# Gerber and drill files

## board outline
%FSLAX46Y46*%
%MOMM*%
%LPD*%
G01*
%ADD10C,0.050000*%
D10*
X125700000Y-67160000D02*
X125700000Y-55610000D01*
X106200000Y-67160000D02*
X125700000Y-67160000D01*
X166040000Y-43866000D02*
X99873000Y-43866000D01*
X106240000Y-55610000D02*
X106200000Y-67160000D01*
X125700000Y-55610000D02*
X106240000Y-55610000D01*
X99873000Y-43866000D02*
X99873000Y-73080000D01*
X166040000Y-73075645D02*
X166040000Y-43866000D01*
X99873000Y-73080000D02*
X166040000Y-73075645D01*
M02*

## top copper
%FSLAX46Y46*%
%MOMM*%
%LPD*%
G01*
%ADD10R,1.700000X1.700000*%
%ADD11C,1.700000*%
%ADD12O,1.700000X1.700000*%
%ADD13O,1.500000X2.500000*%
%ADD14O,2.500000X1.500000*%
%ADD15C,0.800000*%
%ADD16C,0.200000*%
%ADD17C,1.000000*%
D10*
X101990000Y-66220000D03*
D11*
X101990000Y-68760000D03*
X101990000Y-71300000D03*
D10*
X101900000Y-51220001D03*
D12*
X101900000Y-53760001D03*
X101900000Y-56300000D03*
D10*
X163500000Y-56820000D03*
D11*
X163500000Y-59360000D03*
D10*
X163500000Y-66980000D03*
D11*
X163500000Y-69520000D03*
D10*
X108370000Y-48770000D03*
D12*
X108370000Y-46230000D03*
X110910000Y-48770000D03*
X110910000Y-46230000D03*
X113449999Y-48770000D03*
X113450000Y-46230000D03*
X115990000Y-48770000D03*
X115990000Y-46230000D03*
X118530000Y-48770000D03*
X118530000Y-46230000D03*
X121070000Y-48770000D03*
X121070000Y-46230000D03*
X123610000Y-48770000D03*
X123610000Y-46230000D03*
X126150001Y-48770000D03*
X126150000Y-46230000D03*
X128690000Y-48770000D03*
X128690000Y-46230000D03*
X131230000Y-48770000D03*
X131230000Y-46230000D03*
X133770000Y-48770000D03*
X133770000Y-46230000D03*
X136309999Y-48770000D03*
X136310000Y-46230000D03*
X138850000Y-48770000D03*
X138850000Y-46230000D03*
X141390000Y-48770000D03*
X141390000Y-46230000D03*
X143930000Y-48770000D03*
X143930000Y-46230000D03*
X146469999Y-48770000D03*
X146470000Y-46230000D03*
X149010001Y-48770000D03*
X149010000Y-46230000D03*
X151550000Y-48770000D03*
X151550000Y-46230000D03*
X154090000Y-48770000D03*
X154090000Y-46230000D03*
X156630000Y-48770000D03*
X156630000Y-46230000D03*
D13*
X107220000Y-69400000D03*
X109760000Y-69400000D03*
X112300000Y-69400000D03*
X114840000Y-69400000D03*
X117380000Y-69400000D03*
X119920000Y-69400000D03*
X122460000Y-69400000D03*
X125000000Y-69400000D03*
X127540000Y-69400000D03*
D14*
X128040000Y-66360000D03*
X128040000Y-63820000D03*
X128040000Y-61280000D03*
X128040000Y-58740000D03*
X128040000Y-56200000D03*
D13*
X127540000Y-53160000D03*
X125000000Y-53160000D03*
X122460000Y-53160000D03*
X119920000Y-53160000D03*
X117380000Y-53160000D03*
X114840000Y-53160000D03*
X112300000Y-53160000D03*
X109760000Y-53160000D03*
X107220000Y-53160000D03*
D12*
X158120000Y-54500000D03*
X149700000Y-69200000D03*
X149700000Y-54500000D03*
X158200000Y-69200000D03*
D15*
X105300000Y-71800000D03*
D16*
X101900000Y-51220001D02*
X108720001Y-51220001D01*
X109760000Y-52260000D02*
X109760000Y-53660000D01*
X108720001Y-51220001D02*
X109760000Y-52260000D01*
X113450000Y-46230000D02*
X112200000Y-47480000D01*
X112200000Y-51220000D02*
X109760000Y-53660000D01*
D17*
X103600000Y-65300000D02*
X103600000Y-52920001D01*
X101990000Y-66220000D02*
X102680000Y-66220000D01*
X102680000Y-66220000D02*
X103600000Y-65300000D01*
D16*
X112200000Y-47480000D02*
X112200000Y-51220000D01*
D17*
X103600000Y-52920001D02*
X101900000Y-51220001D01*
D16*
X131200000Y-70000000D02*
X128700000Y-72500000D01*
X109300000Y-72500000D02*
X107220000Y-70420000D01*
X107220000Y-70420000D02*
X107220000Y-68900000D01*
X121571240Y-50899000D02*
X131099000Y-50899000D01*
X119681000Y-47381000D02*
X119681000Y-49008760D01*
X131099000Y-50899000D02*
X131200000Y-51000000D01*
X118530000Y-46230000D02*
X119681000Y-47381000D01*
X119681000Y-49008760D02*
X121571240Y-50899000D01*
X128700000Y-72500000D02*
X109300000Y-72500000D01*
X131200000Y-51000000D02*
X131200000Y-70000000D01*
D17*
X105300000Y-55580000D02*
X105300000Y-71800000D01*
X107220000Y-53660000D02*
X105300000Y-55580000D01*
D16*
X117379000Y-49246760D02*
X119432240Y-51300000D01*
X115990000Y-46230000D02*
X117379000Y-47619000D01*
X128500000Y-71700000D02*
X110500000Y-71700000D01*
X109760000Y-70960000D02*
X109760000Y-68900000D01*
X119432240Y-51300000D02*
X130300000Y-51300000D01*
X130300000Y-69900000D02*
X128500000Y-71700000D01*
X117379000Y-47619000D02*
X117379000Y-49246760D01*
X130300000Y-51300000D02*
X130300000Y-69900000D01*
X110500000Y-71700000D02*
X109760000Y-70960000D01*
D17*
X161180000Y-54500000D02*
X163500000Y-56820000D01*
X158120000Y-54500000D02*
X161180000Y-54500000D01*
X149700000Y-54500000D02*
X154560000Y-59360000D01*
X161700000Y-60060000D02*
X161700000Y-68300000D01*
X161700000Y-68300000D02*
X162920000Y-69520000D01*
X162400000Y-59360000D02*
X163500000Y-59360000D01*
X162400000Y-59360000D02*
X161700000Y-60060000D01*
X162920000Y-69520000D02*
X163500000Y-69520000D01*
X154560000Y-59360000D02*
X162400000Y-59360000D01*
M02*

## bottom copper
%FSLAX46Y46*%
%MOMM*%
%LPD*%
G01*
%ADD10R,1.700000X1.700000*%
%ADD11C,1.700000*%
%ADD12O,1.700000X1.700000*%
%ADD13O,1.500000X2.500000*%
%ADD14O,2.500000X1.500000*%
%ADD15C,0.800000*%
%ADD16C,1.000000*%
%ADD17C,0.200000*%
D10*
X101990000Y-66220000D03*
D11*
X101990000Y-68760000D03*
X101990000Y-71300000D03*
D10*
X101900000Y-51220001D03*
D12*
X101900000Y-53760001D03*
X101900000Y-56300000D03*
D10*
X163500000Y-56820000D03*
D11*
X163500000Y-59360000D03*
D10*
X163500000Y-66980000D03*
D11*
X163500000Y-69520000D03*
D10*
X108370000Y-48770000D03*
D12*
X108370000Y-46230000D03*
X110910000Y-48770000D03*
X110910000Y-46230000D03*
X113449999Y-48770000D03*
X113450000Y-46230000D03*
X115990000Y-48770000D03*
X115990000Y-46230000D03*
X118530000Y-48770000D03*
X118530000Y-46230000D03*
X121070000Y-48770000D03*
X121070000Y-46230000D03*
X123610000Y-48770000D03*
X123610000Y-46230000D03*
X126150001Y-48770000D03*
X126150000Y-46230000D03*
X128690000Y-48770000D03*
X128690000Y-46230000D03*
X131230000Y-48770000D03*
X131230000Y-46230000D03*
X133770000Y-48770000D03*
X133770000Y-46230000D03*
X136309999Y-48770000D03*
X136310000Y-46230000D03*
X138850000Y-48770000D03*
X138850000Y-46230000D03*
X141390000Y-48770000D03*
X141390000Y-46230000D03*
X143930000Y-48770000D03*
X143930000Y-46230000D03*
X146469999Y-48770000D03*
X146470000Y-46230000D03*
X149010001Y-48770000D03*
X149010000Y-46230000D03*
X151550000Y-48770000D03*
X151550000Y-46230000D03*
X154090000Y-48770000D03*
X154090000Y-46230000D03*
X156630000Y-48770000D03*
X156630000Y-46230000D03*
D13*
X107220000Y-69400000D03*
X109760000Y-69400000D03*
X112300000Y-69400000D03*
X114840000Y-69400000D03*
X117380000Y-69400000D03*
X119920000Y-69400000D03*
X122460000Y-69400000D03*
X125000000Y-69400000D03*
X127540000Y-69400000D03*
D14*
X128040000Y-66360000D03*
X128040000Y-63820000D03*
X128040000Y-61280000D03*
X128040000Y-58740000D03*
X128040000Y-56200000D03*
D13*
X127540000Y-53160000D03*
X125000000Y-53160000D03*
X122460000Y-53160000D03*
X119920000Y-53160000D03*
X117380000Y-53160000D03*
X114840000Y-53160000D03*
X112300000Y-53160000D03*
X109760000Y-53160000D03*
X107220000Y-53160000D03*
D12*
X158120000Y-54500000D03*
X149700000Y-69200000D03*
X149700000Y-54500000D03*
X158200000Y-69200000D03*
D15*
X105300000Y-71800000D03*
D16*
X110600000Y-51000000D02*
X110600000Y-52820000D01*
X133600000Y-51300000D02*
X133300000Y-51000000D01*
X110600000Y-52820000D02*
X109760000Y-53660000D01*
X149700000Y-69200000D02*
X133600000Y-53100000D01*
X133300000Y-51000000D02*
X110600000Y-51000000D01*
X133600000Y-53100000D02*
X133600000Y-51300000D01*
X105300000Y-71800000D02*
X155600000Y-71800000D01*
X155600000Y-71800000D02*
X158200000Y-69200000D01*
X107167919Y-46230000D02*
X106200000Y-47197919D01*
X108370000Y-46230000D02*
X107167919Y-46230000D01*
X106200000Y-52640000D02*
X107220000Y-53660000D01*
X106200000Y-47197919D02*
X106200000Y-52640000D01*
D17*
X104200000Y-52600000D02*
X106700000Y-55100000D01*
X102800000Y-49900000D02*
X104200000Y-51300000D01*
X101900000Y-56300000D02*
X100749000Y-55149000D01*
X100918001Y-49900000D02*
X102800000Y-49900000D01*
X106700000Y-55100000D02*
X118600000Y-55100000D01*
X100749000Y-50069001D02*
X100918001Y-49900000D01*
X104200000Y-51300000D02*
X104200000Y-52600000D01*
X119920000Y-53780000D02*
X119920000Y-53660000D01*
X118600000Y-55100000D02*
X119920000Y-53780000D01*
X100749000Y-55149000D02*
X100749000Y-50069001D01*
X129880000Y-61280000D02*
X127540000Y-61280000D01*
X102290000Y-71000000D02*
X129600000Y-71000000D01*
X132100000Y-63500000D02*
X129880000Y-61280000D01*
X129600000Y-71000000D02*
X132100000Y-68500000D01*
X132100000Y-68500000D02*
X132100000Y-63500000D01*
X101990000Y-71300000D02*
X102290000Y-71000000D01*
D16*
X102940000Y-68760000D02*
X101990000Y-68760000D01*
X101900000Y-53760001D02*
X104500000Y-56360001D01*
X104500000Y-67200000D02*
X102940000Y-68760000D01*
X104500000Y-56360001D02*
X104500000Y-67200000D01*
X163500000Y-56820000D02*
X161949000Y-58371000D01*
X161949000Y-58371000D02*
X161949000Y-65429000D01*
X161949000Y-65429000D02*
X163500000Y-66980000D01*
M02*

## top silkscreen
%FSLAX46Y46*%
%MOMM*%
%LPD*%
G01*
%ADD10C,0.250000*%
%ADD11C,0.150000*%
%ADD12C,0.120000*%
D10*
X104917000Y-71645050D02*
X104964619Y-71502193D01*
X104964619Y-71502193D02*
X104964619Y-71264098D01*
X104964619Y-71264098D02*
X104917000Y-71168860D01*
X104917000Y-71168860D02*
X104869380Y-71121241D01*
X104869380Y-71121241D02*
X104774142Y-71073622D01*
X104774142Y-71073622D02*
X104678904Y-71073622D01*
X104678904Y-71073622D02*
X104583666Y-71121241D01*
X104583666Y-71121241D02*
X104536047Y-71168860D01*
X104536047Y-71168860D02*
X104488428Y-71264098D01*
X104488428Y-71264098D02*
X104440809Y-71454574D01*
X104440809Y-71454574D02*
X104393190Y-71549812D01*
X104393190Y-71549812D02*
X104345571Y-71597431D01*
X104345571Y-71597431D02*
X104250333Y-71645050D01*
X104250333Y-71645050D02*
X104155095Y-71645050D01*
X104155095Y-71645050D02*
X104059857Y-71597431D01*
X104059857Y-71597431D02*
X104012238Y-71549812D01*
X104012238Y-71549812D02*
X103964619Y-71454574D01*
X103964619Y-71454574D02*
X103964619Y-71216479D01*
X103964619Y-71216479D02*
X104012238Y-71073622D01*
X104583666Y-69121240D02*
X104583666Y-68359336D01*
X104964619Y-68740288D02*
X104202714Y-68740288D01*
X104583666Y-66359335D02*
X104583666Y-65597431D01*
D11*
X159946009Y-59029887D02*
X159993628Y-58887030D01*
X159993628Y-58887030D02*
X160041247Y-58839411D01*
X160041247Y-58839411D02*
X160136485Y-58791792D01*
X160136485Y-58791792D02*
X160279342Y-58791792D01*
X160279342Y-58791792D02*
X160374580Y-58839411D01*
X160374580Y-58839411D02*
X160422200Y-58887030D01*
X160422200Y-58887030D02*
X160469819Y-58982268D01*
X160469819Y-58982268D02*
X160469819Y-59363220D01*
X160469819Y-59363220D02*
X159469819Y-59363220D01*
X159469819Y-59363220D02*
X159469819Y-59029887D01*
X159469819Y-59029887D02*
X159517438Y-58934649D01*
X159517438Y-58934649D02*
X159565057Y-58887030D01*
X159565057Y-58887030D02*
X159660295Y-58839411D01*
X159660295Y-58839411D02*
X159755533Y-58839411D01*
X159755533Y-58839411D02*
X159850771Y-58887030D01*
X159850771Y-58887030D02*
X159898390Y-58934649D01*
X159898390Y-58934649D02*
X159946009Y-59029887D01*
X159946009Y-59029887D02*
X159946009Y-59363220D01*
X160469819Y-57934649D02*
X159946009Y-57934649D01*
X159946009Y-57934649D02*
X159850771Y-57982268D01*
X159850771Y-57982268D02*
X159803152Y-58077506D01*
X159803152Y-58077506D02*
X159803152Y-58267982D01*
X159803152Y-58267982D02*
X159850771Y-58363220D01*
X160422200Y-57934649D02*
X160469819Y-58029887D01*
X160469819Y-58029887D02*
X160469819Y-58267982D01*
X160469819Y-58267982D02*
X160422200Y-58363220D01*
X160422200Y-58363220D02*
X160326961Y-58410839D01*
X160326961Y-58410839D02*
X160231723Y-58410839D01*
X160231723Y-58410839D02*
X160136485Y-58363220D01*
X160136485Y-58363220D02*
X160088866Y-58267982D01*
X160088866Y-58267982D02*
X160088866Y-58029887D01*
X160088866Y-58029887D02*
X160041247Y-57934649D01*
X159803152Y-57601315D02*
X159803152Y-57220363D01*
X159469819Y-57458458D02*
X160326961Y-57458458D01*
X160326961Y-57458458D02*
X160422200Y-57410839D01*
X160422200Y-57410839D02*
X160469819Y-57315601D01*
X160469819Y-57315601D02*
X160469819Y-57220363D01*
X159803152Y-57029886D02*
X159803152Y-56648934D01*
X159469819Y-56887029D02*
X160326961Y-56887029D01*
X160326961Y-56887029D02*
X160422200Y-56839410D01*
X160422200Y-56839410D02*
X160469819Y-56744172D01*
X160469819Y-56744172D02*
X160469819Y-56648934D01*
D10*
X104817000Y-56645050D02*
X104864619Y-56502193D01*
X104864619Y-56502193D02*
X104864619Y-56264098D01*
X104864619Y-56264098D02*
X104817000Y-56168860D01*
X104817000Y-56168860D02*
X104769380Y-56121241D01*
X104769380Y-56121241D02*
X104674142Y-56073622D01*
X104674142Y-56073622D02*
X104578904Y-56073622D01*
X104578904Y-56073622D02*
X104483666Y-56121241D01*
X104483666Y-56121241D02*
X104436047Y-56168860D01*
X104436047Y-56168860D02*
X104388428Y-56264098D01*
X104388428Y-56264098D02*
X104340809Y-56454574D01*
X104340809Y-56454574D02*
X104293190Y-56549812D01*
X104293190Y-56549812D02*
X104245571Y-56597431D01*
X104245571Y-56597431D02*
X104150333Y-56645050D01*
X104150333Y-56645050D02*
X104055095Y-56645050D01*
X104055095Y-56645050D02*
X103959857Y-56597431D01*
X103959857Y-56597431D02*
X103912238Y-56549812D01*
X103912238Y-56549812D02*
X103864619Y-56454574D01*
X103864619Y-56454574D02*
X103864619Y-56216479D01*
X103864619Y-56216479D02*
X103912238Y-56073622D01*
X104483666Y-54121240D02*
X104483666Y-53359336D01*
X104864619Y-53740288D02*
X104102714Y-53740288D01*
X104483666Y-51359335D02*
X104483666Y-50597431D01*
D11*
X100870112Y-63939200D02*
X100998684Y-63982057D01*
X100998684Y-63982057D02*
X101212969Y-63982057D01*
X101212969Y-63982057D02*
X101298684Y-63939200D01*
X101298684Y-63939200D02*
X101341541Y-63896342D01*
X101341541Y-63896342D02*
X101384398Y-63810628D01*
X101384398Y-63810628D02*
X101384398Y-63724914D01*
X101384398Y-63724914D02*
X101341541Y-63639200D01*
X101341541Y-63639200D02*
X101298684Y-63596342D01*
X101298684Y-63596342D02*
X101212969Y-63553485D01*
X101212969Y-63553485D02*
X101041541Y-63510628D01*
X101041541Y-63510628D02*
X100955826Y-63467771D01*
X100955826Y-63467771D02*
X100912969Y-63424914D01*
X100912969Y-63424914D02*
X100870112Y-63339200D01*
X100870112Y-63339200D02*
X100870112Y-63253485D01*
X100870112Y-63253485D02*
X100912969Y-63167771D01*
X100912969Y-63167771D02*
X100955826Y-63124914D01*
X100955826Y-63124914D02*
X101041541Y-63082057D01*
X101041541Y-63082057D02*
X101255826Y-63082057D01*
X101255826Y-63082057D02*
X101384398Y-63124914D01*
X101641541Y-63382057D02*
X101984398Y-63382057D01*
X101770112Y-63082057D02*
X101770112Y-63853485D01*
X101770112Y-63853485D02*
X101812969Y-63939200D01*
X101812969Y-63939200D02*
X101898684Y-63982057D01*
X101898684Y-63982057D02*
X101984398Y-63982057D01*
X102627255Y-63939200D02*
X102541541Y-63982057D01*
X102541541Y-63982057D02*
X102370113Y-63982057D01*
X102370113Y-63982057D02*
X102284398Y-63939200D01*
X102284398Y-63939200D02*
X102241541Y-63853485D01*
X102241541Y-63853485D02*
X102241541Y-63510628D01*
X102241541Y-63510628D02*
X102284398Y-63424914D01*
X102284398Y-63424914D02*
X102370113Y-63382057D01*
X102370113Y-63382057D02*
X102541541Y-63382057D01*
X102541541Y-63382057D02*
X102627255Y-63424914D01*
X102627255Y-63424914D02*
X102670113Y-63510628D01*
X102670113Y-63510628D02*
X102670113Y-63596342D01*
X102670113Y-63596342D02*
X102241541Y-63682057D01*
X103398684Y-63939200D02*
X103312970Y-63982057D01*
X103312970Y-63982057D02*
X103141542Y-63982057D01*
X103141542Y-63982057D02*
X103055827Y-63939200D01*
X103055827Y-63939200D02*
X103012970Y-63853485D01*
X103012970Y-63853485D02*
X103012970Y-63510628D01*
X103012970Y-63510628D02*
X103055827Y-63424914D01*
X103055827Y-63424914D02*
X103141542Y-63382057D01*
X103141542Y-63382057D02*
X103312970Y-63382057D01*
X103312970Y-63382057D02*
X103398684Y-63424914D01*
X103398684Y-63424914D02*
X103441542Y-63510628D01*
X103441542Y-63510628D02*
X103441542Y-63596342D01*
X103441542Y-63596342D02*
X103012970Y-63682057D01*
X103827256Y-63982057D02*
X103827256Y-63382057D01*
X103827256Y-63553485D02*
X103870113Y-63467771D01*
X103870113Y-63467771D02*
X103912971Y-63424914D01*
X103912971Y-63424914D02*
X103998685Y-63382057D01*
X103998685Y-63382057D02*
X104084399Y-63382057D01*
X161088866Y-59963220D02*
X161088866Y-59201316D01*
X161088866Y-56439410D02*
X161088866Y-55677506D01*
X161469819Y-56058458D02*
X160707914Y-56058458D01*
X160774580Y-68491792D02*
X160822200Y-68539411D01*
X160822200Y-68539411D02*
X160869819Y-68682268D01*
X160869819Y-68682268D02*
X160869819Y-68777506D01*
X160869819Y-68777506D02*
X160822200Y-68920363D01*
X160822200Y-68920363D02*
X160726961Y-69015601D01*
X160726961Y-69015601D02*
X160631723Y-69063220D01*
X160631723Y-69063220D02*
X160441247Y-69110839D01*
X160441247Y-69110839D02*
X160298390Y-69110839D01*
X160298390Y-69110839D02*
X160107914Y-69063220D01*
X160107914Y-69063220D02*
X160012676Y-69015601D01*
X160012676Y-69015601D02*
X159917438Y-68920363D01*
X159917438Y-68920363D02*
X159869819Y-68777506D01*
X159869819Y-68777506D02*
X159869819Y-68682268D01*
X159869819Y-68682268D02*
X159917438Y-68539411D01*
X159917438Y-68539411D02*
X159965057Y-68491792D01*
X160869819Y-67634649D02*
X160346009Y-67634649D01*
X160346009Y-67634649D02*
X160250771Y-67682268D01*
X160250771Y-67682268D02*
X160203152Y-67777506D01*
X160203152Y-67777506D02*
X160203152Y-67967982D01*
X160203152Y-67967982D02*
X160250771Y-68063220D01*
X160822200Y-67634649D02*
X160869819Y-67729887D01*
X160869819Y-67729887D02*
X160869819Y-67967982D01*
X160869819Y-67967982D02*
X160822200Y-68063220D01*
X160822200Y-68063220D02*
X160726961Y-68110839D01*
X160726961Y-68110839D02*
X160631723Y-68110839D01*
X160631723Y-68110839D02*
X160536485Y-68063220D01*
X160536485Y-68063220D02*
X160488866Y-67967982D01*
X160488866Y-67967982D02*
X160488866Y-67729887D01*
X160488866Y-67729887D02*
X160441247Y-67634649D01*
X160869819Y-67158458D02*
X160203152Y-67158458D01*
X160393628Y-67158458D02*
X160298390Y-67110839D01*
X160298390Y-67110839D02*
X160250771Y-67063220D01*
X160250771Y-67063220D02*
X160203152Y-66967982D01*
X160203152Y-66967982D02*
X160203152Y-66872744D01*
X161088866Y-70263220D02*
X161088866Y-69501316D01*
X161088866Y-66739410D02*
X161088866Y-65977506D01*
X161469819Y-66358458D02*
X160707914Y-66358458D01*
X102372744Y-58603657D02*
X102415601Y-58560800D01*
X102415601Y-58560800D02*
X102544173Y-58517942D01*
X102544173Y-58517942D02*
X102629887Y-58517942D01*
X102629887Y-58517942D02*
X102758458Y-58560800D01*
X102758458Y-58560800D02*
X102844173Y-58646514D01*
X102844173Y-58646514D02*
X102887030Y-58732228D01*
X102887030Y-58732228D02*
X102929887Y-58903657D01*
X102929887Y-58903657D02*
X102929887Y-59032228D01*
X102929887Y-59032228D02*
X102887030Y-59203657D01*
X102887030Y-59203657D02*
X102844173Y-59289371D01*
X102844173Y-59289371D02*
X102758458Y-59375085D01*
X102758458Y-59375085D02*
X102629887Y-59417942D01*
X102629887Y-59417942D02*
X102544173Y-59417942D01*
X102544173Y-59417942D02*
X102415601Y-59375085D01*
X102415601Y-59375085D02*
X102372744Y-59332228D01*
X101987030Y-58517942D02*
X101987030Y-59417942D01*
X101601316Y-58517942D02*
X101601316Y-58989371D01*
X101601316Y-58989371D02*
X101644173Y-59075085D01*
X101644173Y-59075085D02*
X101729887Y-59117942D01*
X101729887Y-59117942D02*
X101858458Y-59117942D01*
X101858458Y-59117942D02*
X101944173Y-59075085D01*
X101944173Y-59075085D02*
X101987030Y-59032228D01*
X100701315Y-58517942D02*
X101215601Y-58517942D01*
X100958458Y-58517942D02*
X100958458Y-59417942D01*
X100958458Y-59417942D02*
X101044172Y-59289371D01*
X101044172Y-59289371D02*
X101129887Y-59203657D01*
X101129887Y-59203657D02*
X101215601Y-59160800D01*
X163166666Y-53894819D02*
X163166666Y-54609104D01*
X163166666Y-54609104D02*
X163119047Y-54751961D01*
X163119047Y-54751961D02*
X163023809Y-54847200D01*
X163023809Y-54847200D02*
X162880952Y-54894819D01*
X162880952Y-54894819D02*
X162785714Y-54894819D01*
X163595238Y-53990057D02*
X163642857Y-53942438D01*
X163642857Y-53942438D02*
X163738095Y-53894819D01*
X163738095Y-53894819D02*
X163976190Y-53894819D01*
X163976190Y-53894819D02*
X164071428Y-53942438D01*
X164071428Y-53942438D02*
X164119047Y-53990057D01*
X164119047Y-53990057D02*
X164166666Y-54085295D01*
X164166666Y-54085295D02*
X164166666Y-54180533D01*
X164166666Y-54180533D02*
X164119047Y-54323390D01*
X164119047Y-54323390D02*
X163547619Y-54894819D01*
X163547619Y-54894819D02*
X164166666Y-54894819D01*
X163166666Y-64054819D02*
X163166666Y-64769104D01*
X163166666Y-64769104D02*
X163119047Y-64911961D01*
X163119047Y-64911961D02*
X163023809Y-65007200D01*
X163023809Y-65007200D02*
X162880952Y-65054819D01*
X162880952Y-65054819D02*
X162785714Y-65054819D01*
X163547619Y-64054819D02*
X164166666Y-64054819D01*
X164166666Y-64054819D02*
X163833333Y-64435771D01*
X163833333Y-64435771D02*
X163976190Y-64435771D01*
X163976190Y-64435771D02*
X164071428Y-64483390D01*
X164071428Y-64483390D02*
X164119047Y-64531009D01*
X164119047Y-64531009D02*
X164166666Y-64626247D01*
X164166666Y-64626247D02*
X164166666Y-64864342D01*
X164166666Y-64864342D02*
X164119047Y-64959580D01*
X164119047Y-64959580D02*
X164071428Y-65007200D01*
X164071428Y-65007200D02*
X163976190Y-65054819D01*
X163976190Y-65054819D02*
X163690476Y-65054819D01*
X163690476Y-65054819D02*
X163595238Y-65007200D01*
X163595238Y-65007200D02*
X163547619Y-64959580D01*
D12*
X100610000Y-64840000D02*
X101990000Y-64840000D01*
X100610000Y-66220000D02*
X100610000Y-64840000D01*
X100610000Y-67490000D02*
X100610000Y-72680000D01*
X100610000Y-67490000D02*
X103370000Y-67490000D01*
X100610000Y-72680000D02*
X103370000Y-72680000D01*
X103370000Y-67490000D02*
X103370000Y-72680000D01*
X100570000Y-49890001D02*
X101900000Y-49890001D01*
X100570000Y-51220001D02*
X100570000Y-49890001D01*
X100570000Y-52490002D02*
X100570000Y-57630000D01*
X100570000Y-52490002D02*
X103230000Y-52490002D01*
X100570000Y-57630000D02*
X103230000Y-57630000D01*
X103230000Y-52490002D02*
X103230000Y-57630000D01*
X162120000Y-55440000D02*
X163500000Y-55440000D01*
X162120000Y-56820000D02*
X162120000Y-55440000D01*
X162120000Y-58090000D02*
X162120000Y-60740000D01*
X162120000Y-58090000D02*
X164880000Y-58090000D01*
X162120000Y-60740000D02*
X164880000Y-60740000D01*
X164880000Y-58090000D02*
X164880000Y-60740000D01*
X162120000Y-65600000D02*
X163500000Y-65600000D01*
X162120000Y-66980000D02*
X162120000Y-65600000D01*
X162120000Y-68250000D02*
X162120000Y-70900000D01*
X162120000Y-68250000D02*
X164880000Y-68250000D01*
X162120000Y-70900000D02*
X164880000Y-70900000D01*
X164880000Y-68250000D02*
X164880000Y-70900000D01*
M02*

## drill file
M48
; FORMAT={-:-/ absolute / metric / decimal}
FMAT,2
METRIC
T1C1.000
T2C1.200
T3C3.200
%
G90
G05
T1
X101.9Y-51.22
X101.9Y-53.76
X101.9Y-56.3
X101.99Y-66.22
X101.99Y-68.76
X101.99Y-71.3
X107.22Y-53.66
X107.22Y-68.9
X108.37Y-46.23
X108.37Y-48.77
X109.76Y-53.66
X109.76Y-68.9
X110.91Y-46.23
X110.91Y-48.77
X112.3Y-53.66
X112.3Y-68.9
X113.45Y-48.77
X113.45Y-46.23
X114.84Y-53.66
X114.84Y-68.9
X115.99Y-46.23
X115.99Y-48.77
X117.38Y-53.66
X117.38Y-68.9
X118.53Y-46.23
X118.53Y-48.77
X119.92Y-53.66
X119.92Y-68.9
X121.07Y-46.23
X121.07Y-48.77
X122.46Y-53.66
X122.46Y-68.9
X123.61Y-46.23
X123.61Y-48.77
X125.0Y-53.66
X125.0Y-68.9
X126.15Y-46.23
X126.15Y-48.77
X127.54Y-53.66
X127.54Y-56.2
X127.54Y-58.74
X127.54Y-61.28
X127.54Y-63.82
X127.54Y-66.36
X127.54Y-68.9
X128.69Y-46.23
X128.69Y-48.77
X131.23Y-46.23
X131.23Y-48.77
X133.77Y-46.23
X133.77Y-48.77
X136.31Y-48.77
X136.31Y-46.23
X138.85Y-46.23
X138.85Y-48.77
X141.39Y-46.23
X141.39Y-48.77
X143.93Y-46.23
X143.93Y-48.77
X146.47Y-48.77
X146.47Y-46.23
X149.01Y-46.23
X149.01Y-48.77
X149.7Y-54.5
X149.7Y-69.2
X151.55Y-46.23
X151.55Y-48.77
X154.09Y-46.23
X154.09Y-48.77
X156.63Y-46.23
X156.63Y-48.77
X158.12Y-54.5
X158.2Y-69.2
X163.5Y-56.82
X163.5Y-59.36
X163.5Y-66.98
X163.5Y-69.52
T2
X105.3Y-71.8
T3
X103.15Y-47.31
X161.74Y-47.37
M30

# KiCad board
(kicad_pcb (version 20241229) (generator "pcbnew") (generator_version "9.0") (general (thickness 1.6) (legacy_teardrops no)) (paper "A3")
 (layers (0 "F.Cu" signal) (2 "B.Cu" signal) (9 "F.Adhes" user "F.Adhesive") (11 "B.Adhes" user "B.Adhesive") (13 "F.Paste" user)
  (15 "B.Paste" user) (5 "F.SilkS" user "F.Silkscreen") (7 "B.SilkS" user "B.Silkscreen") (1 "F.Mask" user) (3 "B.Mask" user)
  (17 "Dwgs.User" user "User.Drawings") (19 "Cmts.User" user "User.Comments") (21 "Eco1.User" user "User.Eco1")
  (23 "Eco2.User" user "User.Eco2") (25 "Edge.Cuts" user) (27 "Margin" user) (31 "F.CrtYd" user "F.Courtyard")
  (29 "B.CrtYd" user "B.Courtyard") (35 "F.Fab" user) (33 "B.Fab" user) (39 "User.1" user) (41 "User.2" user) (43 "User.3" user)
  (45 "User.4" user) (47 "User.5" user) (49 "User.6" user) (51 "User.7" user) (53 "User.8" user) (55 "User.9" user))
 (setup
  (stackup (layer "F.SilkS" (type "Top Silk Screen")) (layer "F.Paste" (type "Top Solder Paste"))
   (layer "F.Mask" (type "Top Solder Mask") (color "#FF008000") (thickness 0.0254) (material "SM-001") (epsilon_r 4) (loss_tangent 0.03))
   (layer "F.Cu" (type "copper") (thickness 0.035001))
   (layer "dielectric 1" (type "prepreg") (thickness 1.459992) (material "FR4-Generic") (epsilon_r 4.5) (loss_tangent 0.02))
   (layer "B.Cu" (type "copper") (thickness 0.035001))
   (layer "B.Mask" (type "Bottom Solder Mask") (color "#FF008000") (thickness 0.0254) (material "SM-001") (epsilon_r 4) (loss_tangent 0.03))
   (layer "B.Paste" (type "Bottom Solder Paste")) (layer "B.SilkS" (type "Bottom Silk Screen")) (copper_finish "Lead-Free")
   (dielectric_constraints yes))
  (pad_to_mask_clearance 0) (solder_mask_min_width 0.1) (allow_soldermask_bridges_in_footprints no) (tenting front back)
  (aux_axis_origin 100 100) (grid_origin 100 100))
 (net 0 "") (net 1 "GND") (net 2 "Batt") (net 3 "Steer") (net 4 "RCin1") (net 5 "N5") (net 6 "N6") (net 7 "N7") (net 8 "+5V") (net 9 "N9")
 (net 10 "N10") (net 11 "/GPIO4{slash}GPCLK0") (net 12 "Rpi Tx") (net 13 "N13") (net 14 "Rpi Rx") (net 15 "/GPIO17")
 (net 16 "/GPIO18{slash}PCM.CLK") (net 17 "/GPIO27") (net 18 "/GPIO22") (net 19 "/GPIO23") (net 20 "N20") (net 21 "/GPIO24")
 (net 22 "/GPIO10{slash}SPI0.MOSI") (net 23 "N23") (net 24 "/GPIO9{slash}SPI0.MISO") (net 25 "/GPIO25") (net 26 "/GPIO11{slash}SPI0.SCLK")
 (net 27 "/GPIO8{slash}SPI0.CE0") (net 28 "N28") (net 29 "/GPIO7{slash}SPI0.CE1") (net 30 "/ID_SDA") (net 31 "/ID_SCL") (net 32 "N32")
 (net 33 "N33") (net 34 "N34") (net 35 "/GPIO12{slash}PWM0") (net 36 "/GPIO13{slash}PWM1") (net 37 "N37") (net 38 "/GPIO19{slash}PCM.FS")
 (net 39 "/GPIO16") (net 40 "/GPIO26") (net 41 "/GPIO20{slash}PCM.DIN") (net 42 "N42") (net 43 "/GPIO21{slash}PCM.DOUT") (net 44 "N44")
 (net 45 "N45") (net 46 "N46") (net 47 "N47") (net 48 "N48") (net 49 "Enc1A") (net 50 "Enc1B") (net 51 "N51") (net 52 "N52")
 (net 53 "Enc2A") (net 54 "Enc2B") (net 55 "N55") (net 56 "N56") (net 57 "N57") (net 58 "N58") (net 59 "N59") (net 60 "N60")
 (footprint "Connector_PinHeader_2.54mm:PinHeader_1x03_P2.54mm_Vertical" (layer "F.Cu") (at 101.99 66.22)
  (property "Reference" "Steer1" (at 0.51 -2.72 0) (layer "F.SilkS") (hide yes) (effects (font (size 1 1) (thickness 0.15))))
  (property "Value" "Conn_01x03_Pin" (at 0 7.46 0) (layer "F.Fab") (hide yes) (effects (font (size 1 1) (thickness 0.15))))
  (fp_line (start -1.38 -1.38) (end 0 -1.38) (stroke (width 0.12) (type solid)) (layer "F.SilkS"))
  (fp_line (start -1.38 0) (end -1.38 -1.38) (stroke (width 0.12) (type solid)) (layer "F.SilkS"))
  (fp_line (start -1.38 1.27) (end -1.38 6.46) (stroke (width 0.12) (type solid)) (layer "F.SilkS"))
  (fp_line (start -1.38 1.27) (end 1.38 1.27) (stroke (width 0.12) (type solid)) (layer "F.SilkS"))
  (fp_line (start -1.38 6.46) (end 1.38 6.46) (stroke (width 0.12) (type solid)) (layer "F.SilkS"))
  (fp_line (start 1.38 1.27) (end 1.38 6.46) (stroke (width 0.12) (type solid)) (layer "F.SilkS"))
  (pad "1" thru_hole rect (at 0 0) (size 1.7 1.7) (drill 1) (layers "*.Cu" "*.Mask") (remove_unused_layers no) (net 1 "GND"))
  (pad "2" thru_hole circle (at 0 2.54) (size 1.7 1.7) (drill 1) (layers "*.Cu" "*.Mask") (remove_unused_layers no) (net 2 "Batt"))
  (pad "3" thru_hole circle (at 0 5.08) (size 1.7 1.7) (drill 1) (layers "*.Cu" "*.Mask") (remove_unused_layers no) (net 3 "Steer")))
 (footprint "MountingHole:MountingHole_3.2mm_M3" (layer "F.Cu") (at 103.15 47.31)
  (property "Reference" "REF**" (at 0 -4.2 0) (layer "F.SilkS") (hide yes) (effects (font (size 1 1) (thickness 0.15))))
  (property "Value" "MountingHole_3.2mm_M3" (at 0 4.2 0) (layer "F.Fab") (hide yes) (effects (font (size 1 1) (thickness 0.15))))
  (pad "" np_thru_hole circle (at 0 0) (size 3.2 3.2) (drill 3.2) (layers "*.Cu" "*.Mask")))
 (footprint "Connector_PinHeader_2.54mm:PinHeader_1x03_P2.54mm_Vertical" (layer "F.Cu") (at 101.9 51.220001)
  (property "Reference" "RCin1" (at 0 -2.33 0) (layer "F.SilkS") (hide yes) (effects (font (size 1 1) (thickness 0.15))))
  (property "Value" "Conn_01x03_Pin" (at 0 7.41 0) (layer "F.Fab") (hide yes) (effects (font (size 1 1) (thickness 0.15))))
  (fp_line (start -1.33 -1.33) (end 0 -1.33) (stroke (width 0.12) (type solid)) (layer "F.SilkS"))
  (fp_line (start -1.33 0) (end -1.33 -1.33) (stroke (width 0.12) (type solid)) (layer "F.SilkS"))
  (fp_line (start -1.33 1.270001) (end -1.33 6.409999) (stroke (width 0.12) (type solid)) (layer "F.SilkS"))
  (fp_line (start -1.33 1.270001) (end 1.33 1.270001) (stroke (width 0.12) (type solid)) (layer "F.SilkS"))
  (fp_line (start -1.33 6.409999) (end 1.33 6.409999) (stroke (width 0.12) (type solid)) (layer "F.SilkS"))
  (fp_line (start 1.33 1.270001) (end 1.33 6.409999) (stroke (width 0.12) (type solid)) (layer "F.SilkS"))
  (pad "1" thru_hole rect (at 0 0) (size 1.7 1.7) (drill 1) (layers "*.Cu" "*.Mask") (remove_unused_layers no) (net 1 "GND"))
  (pad "2" thru_hole oval (at 0 2.54) (size 1.7 1.7) (drill 1) (layers "*.Cu" "*.Mask") (remove_unused_layers no) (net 2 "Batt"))
  (pad "3" thru_hole oval (at 0 5.079999) (size 1.7 1.7) (drill 1) (layers "*.Cu" "*.Mask") (remove_unused_layers no) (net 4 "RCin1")))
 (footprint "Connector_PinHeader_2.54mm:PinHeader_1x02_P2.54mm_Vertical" (layer "F.Cu") (at 163.5 56.82)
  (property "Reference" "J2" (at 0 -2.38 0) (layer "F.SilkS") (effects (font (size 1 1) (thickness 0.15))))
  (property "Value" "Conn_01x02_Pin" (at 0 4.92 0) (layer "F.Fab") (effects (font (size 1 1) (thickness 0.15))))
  (fp_line (start -1.38 -1.38) (end 0 -1.38) (stroke (width 0.12) (type solid)) (layer "F.SilkS"))
  (fp_line (start -1.38 0) (end -1.38 -1.38) (stroke (width 0.12) (type solid)) (layer "F.SilkS"))
  (fp_line (start -1.38 1.27) (end -1.38 3.92) (stroke (width 0.12) (type solid)) (layer "F.SilkS"))
  (fp_line (start -1.38 1.27) (end 1.38 1.27) (stroke (width 0.12) (type solid)) (layer "F.SilkS"))
  (fp_line (start -1.38 3.92) (end 1.38 3.92) (stroke (width 0.12) (type solid)) (layer "F.SilkS"))
  (fp_line (start 1.38 1.27) (end 1.38 3.92) (stroke (width 0.12) (type solid)) (layer "F.SilkS"))
  (pad "1" thru_hole rect (at 0 0) (size 1.7 1.7) (drill 1) (layers "*.Cu" "*.Mask") (remove_unused_layers no) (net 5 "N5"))
  (pad "2" thru_hole circle (at 0 2.54) (size 1.7 1.7) (drill 1) (layers "*.Cu" "*.Mask") (remove_unused_layers no) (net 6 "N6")))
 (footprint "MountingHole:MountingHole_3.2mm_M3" (layer "F.Cu") (at 161.74 47.37)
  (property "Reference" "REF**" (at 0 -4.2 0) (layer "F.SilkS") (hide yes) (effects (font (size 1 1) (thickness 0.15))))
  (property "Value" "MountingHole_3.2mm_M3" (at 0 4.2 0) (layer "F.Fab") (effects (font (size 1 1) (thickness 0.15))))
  (pad "" np_thru_hole circle (at 0 0) (size 3.2 3.2) (drill 3.2) (layers "*.Cu" "*.Mask")))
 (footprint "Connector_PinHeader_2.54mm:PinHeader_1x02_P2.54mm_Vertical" (layer "F.Cu") (at 163.5 66.98)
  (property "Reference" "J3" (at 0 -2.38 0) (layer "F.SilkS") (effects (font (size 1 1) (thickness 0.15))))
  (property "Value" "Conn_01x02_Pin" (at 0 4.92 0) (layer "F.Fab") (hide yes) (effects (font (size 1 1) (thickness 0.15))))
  (fp_line (start -1.38 -1.38) (end 0 -1.38) (stroke (width 0.12) (type solid)) (layer "F.SilkS"))
  (fp_line (start -1.38 0) (end -1.38 -1.38) (stroke (width 0.12) (type solid)) (layer "F.SilkS"))
  (fp_line (start -1.38 1.27) (end -1.38 3.92) (stroke (width 0.12) (type solid)) (layer "F.SilkS"))
  (fp_line (start -1.38 1.27) (end 1.38 1.27) (stroke (width 0.12) (type solid)) (layer "F.SilkS"))
  (fp_line (start -1.38 3.92) (end 1.38 3.92) (stroke (width 0.12) (type solid)) (layer "F.SilkS"))
  (fp_line (start 1.38 1.27) (end 1.38 3.92) (stroke (width 0.12) (type solid)) (layer "F.SilkS"))
  (pad "1" thru_hole rect (at 0 0) (size 1.7 1.7) (drill 1) (layers "*.Cu" "*.Mask") (remove_unused_layers no) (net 5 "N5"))
  (pad "2" thru_hole circle (at 0 2.54) (size 1.7 1.7) (drill 1) (layers "*.Cu" "*.Mask") (remove_unused_layers no) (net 6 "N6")))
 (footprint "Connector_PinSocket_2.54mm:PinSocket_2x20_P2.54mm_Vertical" (layer "B.Cu") (at 108.37 48.77 -90)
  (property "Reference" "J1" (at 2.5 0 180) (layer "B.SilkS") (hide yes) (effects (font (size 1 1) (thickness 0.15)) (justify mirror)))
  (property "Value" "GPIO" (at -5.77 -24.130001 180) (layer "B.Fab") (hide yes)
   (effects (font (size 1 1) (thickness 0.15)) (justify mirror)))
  (pad "1" thru_hole rect (at 0 0 270) (size 1.7 1.7) (drill 1) (layers "*.Cu" "*.Mask") (remove_unused_layers no) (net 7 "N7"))
  (pad "2" thru_hole oval (at -2.54 0 270) (size 1.7 1.7) (drill 1) (layers "*.Cu" "*.Mask") (remove_unused_layers no) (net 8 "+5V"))
  (pad "3" thru_hole oval (at 0 -2.54 270) (size 1.7 1.7) (drill 1) (layers "*.Cu" "*.Mask") (remove_unused_layers no) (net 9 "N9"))
  (pad "4" thru_hole oval (at -2.54 -2.54 270) (size 1.7 1.7) (drill 1) (layers "*.Cu" "*.Mask") (remove_unused_layers no) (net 8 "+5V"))
  (pad "5" thru_hole oval (at 0 -5.079999 270) (size 1.7 1.7) (drill 1) (layers "*.Cu" "*.Mask") (remove_unused_layers no) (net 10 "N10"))
  (pad "6" thru_hole oval (at -2.54 -5.08 270) (size 1.7 1.7) (drill 1) (layers "*.Cu" "*.Mask") (remove_unused_layers no) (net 1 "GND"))
  (pad "7" thru_hole oval (at 0 -7.62 270) (size 1.7 1.7) (drill 1) (layers "*.Cu" "*.Mask") (remove_unused_layers no)
   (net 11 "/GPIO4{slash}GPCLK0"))
  (pad "8" thru_hole oval (at -2.54 -7.62 270) (size 1.7 1.7) (drill 1) (layers "*.Cu" "*.Mask") (remove_unused_layers no) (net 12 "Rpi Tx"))
  (pad "9" thru_hole oval (at 0 -10.16 270) (size 1.7 1.7) (drill 1) (layers "*.Cu" "*.Mask") (remove_unused_layers no) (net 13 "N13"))
  (pad "10" thru_hole oval (at -2.54 -10.16 270) (size 1.7 1.7) (drill 1) (layers "*.Cu" "*.Mask") (remove_unused_layers no)
   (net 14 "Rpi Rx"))
  (pad "11" thru_hole oval (at 0 -12.7 270) (size 1.7 1.7) (drill 1) (layers "*.Cu" "*.Mask") (remove_unused_layers no) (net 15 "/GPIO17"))
  (pad "12" thru_hole oval (at -2.54 -12.7 270) (size 1.7 1.7) (drill 1) (layers "*.Cu" "*.Mask") (remove_unused_layers no)
   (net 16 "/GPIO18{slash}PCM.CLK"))
  (pad "13" thru_hole oval (at 0 -15.24 270) (size 1.7 1.7) (drill 1) (layers "*.Cu" "*.Mask") (remove_unused_layers no) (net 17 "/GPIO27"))
  (pad "14" thru_hole oval (at -2.54 -15.24 270) (size 1.7 1.7) (drill 1) (layers "*.Cu" "*.Mask") (remove_unused_layers no) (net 1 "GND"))
  (pad "15" thru_hole oval (at 0 -17.780001 270) (size 1.7 1.7) (drill 1) (layers "*.Cu" "*.Mask") (remove_unused_layers no)
   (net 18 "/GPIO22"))
  (pad "16" thru_hole oval (at -2.54 -17.78 270) (size 1.7 1.7) (drill 1) (layers "*.Cu" "*.Mask") (remove_unused_layers no)
   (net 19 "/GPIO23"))
  (pad "17" thru_hole oval (at 0 -20.32 270) (size 1.7 1.7) (drill 1) (layers "*.Cu" "*.Mask") (remove_unused_layers no) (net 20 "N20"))
  (pad "18" thru_hole oval (at -2.54 -20.32 270) (size 1.7 1.7) (drill 1) (layers "*.Cu" "*.Mask") (remove_unused_layers no)
   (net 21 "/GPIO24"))
  (pad "19" thru_hole oval (at 0 -22.86 270) (size 1.7 1.7) (drill 1) (layers "*.Cu" "*.Mask") (remove_unused_layers no)
   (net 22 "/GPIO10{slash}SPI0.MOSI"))
  (pad "20" thru_hole oval (at -2.54 -22.86 270) (size 1.7 1.7) (drill 1) (layers "*.Cu" "*.Mask") (remove_unused_layers no) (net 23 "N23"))
  (pad "21" thru_hole oval (at 0 -25.4 270) (size 1.7 1.7) (drill 1) (layers "*.Cu" "*.Mask") (remove_unused_layers no)
   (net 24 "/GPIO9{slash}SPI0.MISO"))
  (pad "22" thru_hole oval (at -2.54 -25.4 270) (size 1.7 1.7) (drill 1) (layers "*.Cu" "*.Mask") (remove_unused_layers no)
   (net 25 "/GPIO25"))
  (pad "23" thru_hole oval (at 0 -27.939999 270) (size 1.7 1.7) (drill 1) (layers "*.Cu" "*.Mask") (remove_unused_layers no)
   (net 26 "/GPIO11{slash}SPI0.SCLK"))
  (pad "24" thru_hole oval (at -2.54 -27.94 270) (size 1.7 1.7) (drill 1) (layers "*.Cu" "*.Mask") (remove_unused_layers no)
   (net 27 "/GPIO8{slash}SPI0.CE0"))
  (pad "25" thru_hole oval (at 0 -30.48 270) (size 1.7 1.7) (drill 1) (layers "*.Cu" "*.Mask") (remove_unused_layers no) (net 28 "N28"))
  (pad "26" thru_hole oval (at -2.54 -30.48 270) (size 1.7 1.7) (drill 1) (layers "*.Cu" "*.Mask") (remove_unused_layers no)
   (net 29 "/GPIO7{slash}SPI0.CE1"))
  (pad "27" thru_hole oval (at 0 -33.02 270) (size 1.7 1.7) (drill 1) (layers "*.Cu" "*.Mask") (remove_unused_layers no) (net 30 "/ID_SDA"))
  (pad "28" thru_hole oval (at -2.54 -33.02 270) (size 1.7 1.7) (drill 1) (layers "*.Cu" "*.Mask") (remove_unused_layers no)
   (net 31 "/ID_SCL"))
  (pad "29" thru_hole oval (at 0 -35.56 270) (size 1.7 1.7) (drill 1) (layers "*.Cu" "*.Mask") (remove_unused_layers no) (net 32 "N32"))
  (pad "30" thru_hole oval (at -2.54 -35.56 270) (size 1.7 1.7) (drill 1) (layers "*.Cu" "*.Mask") (remove_unused_layers no) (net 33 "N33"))
  (pad "31" thru_hole oval (at 0 -38.099999 270) (size 1.7 1.7) (drill 1) (layers "*.Cu" "*.Mask") (remove_unused_layers no) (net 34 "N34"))
  (pad "32" thru_hole oval (at -2.54 -38.1 270) (size 1.7 1.7) (drill 1) (layers "*.Cu" "*.Mask") (remove_unused_layers no)
   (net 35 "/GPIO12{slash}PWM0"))
  (pad "33" thru_hole oval (at 0 -40.640001 270) (size 1.7 1.7) (drill 1) (layers "*.Cu" "*.Mask") (remove_unused_layers no)
   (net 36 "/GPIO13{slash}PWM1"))
  (pad "34" thru_hole oval (at -2.54 -40.64 270) (size 1.7 1.7) (drill 1) (layers "*.Cu" "*.Mask") (remove_unused_layers no) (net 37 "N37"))
  (pad "35" thru_hole oval (at 0 -43.18 270) (size 1.7 1.7) (drill 1) (layers "*.Cu" "*.Mask") (remove_unused_layers no)
   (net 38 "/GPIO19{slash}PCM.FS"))
  (pad "36" thru_hole oval (at -2.54 -43.18 270) (size 1.7 1.7) (drill 1) (layers "*.Cu" "*.Mask") (remove_unused_layers no)
   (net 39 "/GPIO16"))
  (pad "37" thru_hole oval (at 0 -45.72 270) (size 1.7 1.7) (drill 1) (layers "*.Cu" "*.Mask") (remove_unused_layers no) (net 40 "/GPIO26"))
  (pad "38" thru_hole oval (at -2.54 -45.72 270) (size 1.7 1.7) (drill 1) (layers "*.Cu" "*.Mask") (remove_unused_layers no)
   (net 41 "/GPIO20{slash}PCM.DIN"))
  (pad "39" thru_hole oval (at 0 -48.26 270) (size 1.7 1.7) (drill 1) (layers "*.Cu" "*.Mask") (remove_unused_layers no) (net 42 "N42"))
  (pad "40" thru_hole oval (at -2.54 -48.26 270) (size 1.7 1.7) (drill 1) (layers "*.Cu" "*.Mask") (remove_unused_layers no)
   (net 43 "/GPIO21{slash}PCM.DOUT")))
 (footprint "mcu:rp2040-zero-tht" (layer "B.Cu") (at 117.38 61.28 -90)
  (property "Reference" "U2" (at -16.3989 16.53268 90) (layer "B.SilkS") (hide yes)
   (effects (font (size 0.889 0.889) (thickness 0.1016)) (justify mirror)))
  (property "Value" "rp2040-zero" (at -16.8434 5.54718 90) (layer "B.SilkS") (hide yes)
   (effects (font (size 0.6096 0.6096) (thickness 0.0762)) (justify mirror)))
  (pad "1" thru_hole oval (at 7.62 10.16 90) (size 2.5 1.5) (drill 1 (offset -0.5 0)) (layers "*.Cu" "*.Mask") (remove_unused_layers no)
   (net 14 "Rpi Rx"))
  (pad "2" thru_hole oval (at 7.62 7.62 90) (size 2.5 1.5) (drill 1 (offset -0.5 0)) (layers "*.Cu" "*.Mask") (remove_unused_layers no)
   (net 12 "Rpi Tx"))
  (pad "3" thru_hole oval (at 7.62 5.08 90) (size 2.5 1.5) (drill 1 (offset -0.5 0)) (layers "*.Cu" "*.Mask") (remove_unused_layers no)
   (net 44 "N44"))
  (pad "4" thru_hole oval (at 7.62 2.54 90) (size 2.5 1.5) (drill 1 (offset -0.5 0)) (layers "*.Cu" "*.Mask") (remove_unused_layers no)
   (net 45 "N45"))
  (pad "5" thru_hole oval (at 7.62 0 90) (size 2.5 1.5) (drill 1 (offset -0.5 0)) (layers "*.Cu" "*.Mask") (remove_unused_layers no)
   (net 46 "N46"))
  (pad "6" thru_hole oval (at 7.62 -2.54 90) (size 2.5 1.5) (drill 1 (offset -0.5 0)) (layers "*.Cu" "*.Mask") (remove_unused_layers no)
   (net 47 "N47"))
  (pad "7" thru_hole oval (at 7.62 -5.08 90) (size 2.5 1.5) (drill 1 (offset -0.5 0)) (layers "*.Cu" "*.Mask") (remove_unused_layers no)
   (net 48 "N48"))
  (pad "8" thru_hole oval (at 7.62 -7.62 90) (size 2.5 1.5) (drill 1 (offset -0.5 0)) (layers "*.Cu" "*.Mask") (remove_unused_layers no)
   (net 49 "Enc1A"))
  (pad "9" thru_hole oval (at 7.62 -10.16 90) (size 2.5 1.5) (drill 1 (offset -0.5 0)) (layers "*.Cu" "*.Mask") (remove_unused_layers no)
   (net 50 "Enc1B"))
  (pad "10" thru_hole oval (at 5.08 -10.16 180) (size 2.5 1.5) (drill 1 (offset -0.5 0)) (layers "*.Cu" "*.Mask") (remove_unused_layers no)
   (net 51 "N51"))
  (pad "11" thru_hole oval (at 2.54 -10.16 180) (size 2.5 1.5) (drill 1 (offset -0.5 0)) (layers "*.Cu" "*.Mask") (remove_unused_layers no)
   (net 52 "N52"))
  (pad "12" thru_hole oval (at 0 -10.16 180) (size 2.5 1.5) (drill 1 (offset -0.5 0)) (layers "*.Cu" "*.Mask") (remove_unused_layers no)
   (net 3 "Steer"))
  (pad "13" thru_hole oval (at -2.54 -10.16 180) (size 2.5 1.5) (drill 1 (offset -0.5 0)) (layers "*.Cu" "*.Mask") (remove_unused_layers no)
   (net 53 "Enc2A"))
  (pad "14" thru_hole oval (at -5.08 -10.16 180) (size 2.5 1.5) (drill 1 (offset -0.5 0)) (layers "*.Cu" "*.Mask") (remove_unused_layers no)
   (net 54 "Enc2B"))
  (pad "15" thru_hole oval (at -7.62 -10.16 270) (size 2.5 1.5) (drill 1 (offset -0.5 0)) (layers "*.Cu" "*.Mask") (remove_unused_layers no)
   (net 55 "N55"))
  (pad "16" thru_hole oval (at -7.62 -7.62 270) (size 2.5 1.5) (drill 1 (offset -0.5 0)) (layers "*.Cu" "*.Mask") (remove_unused_layers no)
   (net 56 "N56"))
  (pad "17" thru_hole oval (at -7.62 -5.08 270) (size 2.5 1.5) (drill 1 (offset -0.5 0)) (layers "*.Cu" "*.Mask") (remove_unused_layers no)
   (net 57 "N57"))
  (pad "18" thru_hole oval (at -7.62 -2.54 270) (size 2.5 1.5) (drill 1 (offset -0.5 0)) (layers "*.Cu" "*.Mask") (remove_unused_layers no)
   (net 4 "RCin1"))
  (pad "19" thru_hole oval (at -7.62 0 270) (size 2.5 1.5) (drill 1 (offset -0.5 0)) (layers "*.Cu" "*.Mask") (remove_unused_layers no)
   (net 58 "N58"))
  (pad "20" thru_hole oval (at -7.62 2.54 270) (size 2.5 1.5) (drill 1 (offset -0.5 0)) (layers "*.Cu" "*.Mask") (remove_unused_layers no)
   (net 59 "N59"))
  (pad "21" thru_hole oval (at -7.62 5.08 270) (size 2.5 1.5) (drill 1 (offset -0.5 0)) (layers "*.Cu" "*.Mask") (remove_unused_layers no)
   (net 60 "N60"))
  (pad "22" thru_hole oval (at -7.62 7.62 270) (size 2.5 1.5) (drill 1 (offset -0.5 0)) (layers "*.Cu" "*.Mask") (remove_unused_layers no)
   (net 1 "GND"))
  (pad "23" thru_hole oval (at -7.62 10.16 270) (size 2.5 1.5) (drill 1 (offset -0.5 0)) (layers "*.Cu" "*.Mask") (remove_unused_layers no)
   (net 8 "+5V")))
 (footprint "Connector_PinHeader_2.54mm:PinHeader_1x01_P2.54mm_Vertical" (layer "B.Cu") (at 158.12 54.5)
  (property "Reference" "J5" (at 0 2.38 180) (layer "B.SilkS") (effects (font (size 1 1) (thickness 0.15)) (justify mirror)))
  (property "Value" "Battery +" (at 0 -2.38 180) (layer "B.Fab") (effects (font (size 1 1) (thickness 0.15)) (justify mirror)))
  (pad "1" thru_hole oval (at 0 0) (size 1.7 1.7) (drill 1) (layers "*.Cu" "*.Mask") (remove_unused_layers no) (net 5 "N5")))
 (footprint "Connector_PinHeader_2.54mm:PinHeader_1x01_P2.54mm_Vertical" (layer "B.Cu") (at 149.7 69.2)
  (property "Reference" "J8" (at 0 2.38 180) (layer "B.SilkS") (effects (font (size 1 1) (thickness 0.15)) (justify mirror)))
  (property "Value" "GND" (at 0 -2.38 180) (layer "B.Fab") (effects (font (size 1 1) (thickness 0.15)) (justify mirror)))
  (pad "1" thru_hole oval (at 0 0) (size 1.7 1.7) (drill 1) (layers "*.Cu" "*.Mask") (remove_unused_layers no) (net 1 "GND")))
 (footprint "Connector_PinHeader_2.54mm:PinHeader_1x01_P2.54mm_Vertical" (layer "B.Cu") (at 149.7 54.5)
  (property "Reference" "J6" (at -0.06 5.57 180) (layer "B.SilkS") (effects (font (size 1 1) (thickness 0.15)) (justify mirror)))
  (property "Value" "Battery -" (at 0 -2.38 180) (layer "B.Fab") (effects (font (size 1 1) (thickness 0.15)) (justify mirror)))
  (pad "1" thru_hole oval (at 0 0) (size 1.7 1.7) (drill 1) (layers "*.Cu" "*.Mask") (remove_unused_layers no) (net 6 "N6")))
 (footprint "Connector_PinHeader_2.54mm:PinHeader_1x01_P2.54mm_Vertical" (layer "B.Cu") (at 158.2 69.2)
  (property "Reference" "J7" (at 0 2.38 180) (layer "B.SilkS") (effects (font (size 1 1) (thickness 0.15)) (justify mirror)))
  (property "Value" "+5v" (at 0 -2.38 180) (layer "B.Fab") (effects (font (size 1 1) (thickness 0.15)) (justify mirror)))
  (pad "" thru_hole oval (at 0 0) (size 1.7 1.7) (drill 1) (layers "*.Cu" "*.Mask") (remove_unused_layers no) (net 8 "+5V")))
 (gr_line (start 125.7 67.16) (end 125.7 55.61) (stroke (width 0.05) (type default)) (layer "Edge.Cuts"))
 (gr_line (start 106.2 67.16) (end 125.7 67.16) (stroke (width 0.05) (type default)) (layer "Edge.Cuts"))
 (gr_line (start 166.04 43.866) (end 99.873 43.866) (stroke (width 0.05) (type default)) (layer "Edge.Cuts"))
 (gr_line (start 106.24 55.61) (end 106.2 67.16) (stroke (width 0.05) (type default)) (layer "Edge.Cuts"))
 (gr_line (start 125.7 55.61) (end 106.24 55.61) (stroke (width 0.05) (type default)) (layer "Edge.Cuts"))
 (gr_line (start 99.873 43.866) (end 99.873 73.08) (stroke (width 0.05) (type default)) (layer "Edge.Cuts"))
 (gr_line (start 166.04 73.075645) (end 166.04 43.866) (stroke (width 0.05) (type default)) (layer "Edge.Cuts"))
 (gr_line (start 99.873 73.08) (end 166.04 73.075645) (stroke (width 0.05) (type default)) (layer "Edge.Cuts"))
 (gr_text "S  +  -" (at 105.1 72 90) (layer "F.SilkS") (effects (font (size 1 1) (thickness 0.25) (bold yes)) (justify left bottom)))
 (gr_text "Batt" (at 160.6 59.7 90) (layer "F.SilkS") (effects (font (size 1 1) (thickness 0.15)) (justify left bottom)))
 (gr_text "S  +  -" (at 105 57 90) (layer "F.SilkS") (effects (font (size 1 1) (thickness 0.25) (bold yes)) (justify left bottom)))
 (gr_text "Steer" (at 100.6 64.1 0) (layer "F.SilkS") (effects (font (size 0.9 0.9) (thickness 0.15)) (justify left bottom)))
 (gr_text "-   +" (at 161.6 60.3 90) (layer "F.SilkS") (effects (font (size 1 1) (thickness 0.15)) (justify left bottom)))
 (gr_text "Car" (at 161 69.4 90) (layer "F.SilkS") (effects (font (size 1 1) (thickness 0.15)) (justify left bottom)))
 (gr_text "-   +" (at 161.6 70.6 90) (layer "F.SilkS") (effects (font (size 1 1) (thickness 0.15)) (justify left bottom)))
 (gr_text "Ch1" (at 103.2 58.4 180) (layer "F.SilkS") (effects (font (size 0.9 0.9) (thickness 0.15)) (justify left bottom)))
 (segment (start 101.9 51.220001) (end 108.720001 51.220001) (width 0.2) (layer "F.Cu") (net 1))
 (segment (start 109.76 52.26) (end 109.76 53.66) (width 0.2) (layer "F.Cu") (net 1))
 (segment (start 108.720001 51.220001) (end 109.76 52.26) (width 0.2) (layer "F.Cu") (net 1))
 (segment (start 113.45 46.23) (end 112.2 47.48) (width 0.2) (layer "F.Cu") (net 1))
 (segment (start 112.2 51.22) (end 109.76 53.66) (width 0.2) (layer "F.Cu") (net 1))
 (segment (start 103.6 65.3) (end 103.6 52.920001) (width 1) (layer "F.Cu") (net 1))
 (segment (start 101.99 66.22) (end 102.68 66.22) (width 1) (layer "F.Cu") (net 1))
 (segment (start 102.68 66.22) (end 103.6 65.3) (width 1) (layer "F.Cu") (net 1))
 (segment (start 112.2 47.48) (end 112.2 51.22) (width 0.2) (layer "F.Cu") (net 1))
 (segment (start 103.6 52.920001) (end 101.9 51.220001) (width 1) (layer "F.Cu") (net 1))
 (segment (start 110.6 51) (end 110.6 52.82) (width 1) (layer "B.Cu") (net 1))
 (segment (start 133.6 51.3) (end 133.3 51) (width 1) (layer "B.Cu") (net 1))
 (segment (start 110.6 52.82) (end 109.76 53.66) (width 1) (layer "B.Cu") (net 1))
 (segment (start 149.7 69.2) (end 133.6 53.1) (width 1) (layer "B.Cu") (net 1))
 (segment (start 133.3 51) (end 110.6 51) (width 1) (layer "B.Cu") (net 1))
 (segment (start 133.6 53.1) (end 133.6 51.3) (width 1) (layer "B.Cu") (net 1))
 (segment (start 131.2 70) (end 128.7 72.5) (width 0.2) (layer "F.Cu") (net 14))
 (segment (start 109.3 72.5) (end 107.22 70.42) (width 0.2) (layer "F.Cu") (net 14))
 (segment (start 107.22 70.42) (end 107.22 68.9) (width 0.2) (layer "F.Cu") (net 14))
 (segment (start 121.57124 50.899) (end 131.099 50.899) (width 0.2) (layer "F.Cu") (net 14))
 (segment (start 119.681 47.381) (end 119.681 49.00876) (width 0.2) (layer "F.Cu") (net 14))
 (segment (start 131.099 50.899) (end 131.2 51) (width 0.2) (layer "F.Cu") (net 14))
 (segment (start 118.53 46.23) (end 119.681 47.381) (width 0.2) (layer "F.Cu") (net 14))
 (segment (start 119.681 49.00876) (end 121.57124 50.899) (width 0.2) (layer "F.Cu") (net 14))
 (segment (start 128.7 72.5) (end 109.3 72.5) (width 0.2) (layer "F.Cu") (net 14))
 (segment (start 131.2 51) (end 131.2 70) (width 0.2) (layer "F.Cu") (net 14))
 (segment (start 105.3 55.58) (end 105.3 71.8) (width 1) (layer "F.Cu") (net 8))
 (segment (start 107.22 53.66) (end 105.3 55.58) (width 1) (layer "F.Cu") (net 8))
 (via (at 105.3 71.8) (size 0.8) (drill 1.2) (layers "F.Cu" "B.Cu") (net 8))
 (segment (start 105.3 71.8) (end 155.6 71.8) (width 1) (layer "B.Cu") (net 8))
 (segment (start 155.6 71.8) (end 158.2 69.2) (width 1) (layer "B.Cu") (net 8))
 (segment (start 107.167919 46.23) (end 106.2 47.197919) (width 1) (layer "B.Cu") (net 8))
 (segment (start 108.37 46.23) (end 107.167919 46.23) (width 1) (layer "B.Cu") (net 8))
 (segment (start 106.2 52.64) (end 107.22 53.66) (width 1) (layer "B.Cu") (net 8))
 (segment (start 106.2 47.197919) (end 106.2 52.64) (width 1) (layer "B.Cu") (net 8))
 (segment (start 117.379 49.24676) (end 119.43224 51.3) (width 0.2) (layer "F.Cu") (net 12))
 (segment (start 115.99 46.23) (end 117.379 47.619) (width 0.2) (layer "F.Cu") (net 12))
 (segment (start 128.5 71.7) (end 110.5 71.7) (width 0.2) (layer "F.Cu") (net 12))
 (segment (start 109.76 70.96) (end 109.76 68.9) (width 0.2) (layer "F.Cu") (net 12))
 (segment (start 119.43224 51.3) (end 130.3 51.3) (width 0.2) (layer "F.Cu") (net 12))
 (segment (start 130.3 69.9) (end 128.5 71.7) (width 0.2) (layer "F.Cu") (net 12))
 (segment (start 117.379 47.619) (end 117.379 49.24676) (width 0.2) (layer "F.Cu") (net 12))
 (segment (start 130.3 51.3) (end 130.3 69.9) (width 0.2) (layer "F.Cu") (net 12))
 (segment (start 110.5 71.7) (end 109.76 70.96) (width 0.2) (layer "F.Cu") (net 12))
 (segment (start 104.2 52.6) (end 106.7 55.1) (width 0.2) (layer "B.Cu") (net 4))
 (segment (start 102.8 49.9) (end 104.2 51.3) (width 0.2) (layer "B.Cu") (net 4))
 (segment (start 101.9 56.3) (end 100.749 55.149) (width 0.2) (layer "B.Cu") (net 4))
 (segment (start 100.918001 49.9) (end 102.8 49.9) (width 0.2) (layer "B.Cu") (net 4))
 (segment (start 106.7 55.1) (end 118.6 55.1) (width 0.2) (layer "B.Cu") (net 4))
 (segment (start 100.749 50.069001) (end 100.918001 49.9) (width 0.2) (layer "B.Cu") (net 4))
 (segment (start 104.2 51.3) (end 104.2 52.6) (width 0.2) (layer "B.Cu") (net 4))
 (segment (start 119.92 53.78) (end 119.92 53.66) (width 0.2) (layer "B.Cu") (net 4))
 (segment (start 118.6 55.1) (end 119.92 53.78) (width 0.2) (layer "B.Cu") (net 4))
 (segment (start 100.749 55.149) (end 100.749 50.069001) (width 0.2) (layer "B.Cu") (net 4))
 (segment (start 129.88 61.28) (end 127.54 61.28) (width 0.2) (layer "B.Cu") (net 3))
 (segment (start 102.29 71) (end 129.6 71) (width 0.2) (layer "B.Cu") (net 3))
 (segment (start 132.1 63.5) (end 129.88 61.28) (width 0.2) (layer "B.Cu") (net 3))
 (segment (start 129.6 71) (end 132.1 68.5) (width 0.2) (layer "B.Cu") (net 3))
 (segment (start 132.1 68.5) (end 132.1 63.5) (width 0.2) (layer "B.Cu") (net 3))
 (segment (start 101.99 71.3) (end 102.29 71) (width 0.2) (layer "B.Cu") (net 3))
 (segment (start 102.94 68.76) (end 101.99 68.76) (width 1) (layer "B.Cu") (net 2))
 (segment (start 101.9 53.760001) (end 104.5 56.360001) (width 1) (layer "B.Cu") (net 2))
 (segment (start 104.5 67.2) (end 102.94 68.76) (width 1) (layer "B.Cu") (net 2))
 (segment (start 104.5 56.360001) (end 104.5 67.2) (width 1) (layer "B.Cu") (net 2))
 (segment (start 161.18 54.5) (end 163.5 56.82) (width 1) (layer "F.Cu") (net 5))
 (segment (start 158.12 54.5) (end 161.18 54.5) (width 1) (layer "F.Cu") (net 5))
 (segment (start 163.5 56.82) (end 161.949 58.371) (width 1) (layer "B.Cu") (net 5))
 (segment (start 161.949 58.371) (end 161.949 65.429) (width 1) (layer "B.Cu") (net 5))
 (segment (start 161.949 65.429) (end 163.5 66.98) (width 1) (layer "B.Cu") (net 5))
 (segment (start 149.7 54.5) (end 154.56 59.36) (width 1) (layer "F.Cu") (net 6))
 (segment (start 161.7 60.06) (end 161.7 68.3) (width 1) (layer "F.Cu") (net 6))
 (segment (start 161.7 68.3) (end 162.92 69.52) (width 1) (layer "F.Cu") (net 6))
 (segment (start 162.4 59.36) (end 163.5 59.36) (width 1) (layer "F.Cu") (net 6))
 (segment (start 162.4 59.36) (end 161.7 60.06) (width 1) (layer "F.Cu") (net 6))
 (segment (start 162.92 69.52) (end 163.5 69.52) (width 1) (layer "F.Cu") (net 6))
 (segment (start 154.56 59.36) (end 162.4 59.36) (width 1) (layer "F.Cu") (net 6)))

